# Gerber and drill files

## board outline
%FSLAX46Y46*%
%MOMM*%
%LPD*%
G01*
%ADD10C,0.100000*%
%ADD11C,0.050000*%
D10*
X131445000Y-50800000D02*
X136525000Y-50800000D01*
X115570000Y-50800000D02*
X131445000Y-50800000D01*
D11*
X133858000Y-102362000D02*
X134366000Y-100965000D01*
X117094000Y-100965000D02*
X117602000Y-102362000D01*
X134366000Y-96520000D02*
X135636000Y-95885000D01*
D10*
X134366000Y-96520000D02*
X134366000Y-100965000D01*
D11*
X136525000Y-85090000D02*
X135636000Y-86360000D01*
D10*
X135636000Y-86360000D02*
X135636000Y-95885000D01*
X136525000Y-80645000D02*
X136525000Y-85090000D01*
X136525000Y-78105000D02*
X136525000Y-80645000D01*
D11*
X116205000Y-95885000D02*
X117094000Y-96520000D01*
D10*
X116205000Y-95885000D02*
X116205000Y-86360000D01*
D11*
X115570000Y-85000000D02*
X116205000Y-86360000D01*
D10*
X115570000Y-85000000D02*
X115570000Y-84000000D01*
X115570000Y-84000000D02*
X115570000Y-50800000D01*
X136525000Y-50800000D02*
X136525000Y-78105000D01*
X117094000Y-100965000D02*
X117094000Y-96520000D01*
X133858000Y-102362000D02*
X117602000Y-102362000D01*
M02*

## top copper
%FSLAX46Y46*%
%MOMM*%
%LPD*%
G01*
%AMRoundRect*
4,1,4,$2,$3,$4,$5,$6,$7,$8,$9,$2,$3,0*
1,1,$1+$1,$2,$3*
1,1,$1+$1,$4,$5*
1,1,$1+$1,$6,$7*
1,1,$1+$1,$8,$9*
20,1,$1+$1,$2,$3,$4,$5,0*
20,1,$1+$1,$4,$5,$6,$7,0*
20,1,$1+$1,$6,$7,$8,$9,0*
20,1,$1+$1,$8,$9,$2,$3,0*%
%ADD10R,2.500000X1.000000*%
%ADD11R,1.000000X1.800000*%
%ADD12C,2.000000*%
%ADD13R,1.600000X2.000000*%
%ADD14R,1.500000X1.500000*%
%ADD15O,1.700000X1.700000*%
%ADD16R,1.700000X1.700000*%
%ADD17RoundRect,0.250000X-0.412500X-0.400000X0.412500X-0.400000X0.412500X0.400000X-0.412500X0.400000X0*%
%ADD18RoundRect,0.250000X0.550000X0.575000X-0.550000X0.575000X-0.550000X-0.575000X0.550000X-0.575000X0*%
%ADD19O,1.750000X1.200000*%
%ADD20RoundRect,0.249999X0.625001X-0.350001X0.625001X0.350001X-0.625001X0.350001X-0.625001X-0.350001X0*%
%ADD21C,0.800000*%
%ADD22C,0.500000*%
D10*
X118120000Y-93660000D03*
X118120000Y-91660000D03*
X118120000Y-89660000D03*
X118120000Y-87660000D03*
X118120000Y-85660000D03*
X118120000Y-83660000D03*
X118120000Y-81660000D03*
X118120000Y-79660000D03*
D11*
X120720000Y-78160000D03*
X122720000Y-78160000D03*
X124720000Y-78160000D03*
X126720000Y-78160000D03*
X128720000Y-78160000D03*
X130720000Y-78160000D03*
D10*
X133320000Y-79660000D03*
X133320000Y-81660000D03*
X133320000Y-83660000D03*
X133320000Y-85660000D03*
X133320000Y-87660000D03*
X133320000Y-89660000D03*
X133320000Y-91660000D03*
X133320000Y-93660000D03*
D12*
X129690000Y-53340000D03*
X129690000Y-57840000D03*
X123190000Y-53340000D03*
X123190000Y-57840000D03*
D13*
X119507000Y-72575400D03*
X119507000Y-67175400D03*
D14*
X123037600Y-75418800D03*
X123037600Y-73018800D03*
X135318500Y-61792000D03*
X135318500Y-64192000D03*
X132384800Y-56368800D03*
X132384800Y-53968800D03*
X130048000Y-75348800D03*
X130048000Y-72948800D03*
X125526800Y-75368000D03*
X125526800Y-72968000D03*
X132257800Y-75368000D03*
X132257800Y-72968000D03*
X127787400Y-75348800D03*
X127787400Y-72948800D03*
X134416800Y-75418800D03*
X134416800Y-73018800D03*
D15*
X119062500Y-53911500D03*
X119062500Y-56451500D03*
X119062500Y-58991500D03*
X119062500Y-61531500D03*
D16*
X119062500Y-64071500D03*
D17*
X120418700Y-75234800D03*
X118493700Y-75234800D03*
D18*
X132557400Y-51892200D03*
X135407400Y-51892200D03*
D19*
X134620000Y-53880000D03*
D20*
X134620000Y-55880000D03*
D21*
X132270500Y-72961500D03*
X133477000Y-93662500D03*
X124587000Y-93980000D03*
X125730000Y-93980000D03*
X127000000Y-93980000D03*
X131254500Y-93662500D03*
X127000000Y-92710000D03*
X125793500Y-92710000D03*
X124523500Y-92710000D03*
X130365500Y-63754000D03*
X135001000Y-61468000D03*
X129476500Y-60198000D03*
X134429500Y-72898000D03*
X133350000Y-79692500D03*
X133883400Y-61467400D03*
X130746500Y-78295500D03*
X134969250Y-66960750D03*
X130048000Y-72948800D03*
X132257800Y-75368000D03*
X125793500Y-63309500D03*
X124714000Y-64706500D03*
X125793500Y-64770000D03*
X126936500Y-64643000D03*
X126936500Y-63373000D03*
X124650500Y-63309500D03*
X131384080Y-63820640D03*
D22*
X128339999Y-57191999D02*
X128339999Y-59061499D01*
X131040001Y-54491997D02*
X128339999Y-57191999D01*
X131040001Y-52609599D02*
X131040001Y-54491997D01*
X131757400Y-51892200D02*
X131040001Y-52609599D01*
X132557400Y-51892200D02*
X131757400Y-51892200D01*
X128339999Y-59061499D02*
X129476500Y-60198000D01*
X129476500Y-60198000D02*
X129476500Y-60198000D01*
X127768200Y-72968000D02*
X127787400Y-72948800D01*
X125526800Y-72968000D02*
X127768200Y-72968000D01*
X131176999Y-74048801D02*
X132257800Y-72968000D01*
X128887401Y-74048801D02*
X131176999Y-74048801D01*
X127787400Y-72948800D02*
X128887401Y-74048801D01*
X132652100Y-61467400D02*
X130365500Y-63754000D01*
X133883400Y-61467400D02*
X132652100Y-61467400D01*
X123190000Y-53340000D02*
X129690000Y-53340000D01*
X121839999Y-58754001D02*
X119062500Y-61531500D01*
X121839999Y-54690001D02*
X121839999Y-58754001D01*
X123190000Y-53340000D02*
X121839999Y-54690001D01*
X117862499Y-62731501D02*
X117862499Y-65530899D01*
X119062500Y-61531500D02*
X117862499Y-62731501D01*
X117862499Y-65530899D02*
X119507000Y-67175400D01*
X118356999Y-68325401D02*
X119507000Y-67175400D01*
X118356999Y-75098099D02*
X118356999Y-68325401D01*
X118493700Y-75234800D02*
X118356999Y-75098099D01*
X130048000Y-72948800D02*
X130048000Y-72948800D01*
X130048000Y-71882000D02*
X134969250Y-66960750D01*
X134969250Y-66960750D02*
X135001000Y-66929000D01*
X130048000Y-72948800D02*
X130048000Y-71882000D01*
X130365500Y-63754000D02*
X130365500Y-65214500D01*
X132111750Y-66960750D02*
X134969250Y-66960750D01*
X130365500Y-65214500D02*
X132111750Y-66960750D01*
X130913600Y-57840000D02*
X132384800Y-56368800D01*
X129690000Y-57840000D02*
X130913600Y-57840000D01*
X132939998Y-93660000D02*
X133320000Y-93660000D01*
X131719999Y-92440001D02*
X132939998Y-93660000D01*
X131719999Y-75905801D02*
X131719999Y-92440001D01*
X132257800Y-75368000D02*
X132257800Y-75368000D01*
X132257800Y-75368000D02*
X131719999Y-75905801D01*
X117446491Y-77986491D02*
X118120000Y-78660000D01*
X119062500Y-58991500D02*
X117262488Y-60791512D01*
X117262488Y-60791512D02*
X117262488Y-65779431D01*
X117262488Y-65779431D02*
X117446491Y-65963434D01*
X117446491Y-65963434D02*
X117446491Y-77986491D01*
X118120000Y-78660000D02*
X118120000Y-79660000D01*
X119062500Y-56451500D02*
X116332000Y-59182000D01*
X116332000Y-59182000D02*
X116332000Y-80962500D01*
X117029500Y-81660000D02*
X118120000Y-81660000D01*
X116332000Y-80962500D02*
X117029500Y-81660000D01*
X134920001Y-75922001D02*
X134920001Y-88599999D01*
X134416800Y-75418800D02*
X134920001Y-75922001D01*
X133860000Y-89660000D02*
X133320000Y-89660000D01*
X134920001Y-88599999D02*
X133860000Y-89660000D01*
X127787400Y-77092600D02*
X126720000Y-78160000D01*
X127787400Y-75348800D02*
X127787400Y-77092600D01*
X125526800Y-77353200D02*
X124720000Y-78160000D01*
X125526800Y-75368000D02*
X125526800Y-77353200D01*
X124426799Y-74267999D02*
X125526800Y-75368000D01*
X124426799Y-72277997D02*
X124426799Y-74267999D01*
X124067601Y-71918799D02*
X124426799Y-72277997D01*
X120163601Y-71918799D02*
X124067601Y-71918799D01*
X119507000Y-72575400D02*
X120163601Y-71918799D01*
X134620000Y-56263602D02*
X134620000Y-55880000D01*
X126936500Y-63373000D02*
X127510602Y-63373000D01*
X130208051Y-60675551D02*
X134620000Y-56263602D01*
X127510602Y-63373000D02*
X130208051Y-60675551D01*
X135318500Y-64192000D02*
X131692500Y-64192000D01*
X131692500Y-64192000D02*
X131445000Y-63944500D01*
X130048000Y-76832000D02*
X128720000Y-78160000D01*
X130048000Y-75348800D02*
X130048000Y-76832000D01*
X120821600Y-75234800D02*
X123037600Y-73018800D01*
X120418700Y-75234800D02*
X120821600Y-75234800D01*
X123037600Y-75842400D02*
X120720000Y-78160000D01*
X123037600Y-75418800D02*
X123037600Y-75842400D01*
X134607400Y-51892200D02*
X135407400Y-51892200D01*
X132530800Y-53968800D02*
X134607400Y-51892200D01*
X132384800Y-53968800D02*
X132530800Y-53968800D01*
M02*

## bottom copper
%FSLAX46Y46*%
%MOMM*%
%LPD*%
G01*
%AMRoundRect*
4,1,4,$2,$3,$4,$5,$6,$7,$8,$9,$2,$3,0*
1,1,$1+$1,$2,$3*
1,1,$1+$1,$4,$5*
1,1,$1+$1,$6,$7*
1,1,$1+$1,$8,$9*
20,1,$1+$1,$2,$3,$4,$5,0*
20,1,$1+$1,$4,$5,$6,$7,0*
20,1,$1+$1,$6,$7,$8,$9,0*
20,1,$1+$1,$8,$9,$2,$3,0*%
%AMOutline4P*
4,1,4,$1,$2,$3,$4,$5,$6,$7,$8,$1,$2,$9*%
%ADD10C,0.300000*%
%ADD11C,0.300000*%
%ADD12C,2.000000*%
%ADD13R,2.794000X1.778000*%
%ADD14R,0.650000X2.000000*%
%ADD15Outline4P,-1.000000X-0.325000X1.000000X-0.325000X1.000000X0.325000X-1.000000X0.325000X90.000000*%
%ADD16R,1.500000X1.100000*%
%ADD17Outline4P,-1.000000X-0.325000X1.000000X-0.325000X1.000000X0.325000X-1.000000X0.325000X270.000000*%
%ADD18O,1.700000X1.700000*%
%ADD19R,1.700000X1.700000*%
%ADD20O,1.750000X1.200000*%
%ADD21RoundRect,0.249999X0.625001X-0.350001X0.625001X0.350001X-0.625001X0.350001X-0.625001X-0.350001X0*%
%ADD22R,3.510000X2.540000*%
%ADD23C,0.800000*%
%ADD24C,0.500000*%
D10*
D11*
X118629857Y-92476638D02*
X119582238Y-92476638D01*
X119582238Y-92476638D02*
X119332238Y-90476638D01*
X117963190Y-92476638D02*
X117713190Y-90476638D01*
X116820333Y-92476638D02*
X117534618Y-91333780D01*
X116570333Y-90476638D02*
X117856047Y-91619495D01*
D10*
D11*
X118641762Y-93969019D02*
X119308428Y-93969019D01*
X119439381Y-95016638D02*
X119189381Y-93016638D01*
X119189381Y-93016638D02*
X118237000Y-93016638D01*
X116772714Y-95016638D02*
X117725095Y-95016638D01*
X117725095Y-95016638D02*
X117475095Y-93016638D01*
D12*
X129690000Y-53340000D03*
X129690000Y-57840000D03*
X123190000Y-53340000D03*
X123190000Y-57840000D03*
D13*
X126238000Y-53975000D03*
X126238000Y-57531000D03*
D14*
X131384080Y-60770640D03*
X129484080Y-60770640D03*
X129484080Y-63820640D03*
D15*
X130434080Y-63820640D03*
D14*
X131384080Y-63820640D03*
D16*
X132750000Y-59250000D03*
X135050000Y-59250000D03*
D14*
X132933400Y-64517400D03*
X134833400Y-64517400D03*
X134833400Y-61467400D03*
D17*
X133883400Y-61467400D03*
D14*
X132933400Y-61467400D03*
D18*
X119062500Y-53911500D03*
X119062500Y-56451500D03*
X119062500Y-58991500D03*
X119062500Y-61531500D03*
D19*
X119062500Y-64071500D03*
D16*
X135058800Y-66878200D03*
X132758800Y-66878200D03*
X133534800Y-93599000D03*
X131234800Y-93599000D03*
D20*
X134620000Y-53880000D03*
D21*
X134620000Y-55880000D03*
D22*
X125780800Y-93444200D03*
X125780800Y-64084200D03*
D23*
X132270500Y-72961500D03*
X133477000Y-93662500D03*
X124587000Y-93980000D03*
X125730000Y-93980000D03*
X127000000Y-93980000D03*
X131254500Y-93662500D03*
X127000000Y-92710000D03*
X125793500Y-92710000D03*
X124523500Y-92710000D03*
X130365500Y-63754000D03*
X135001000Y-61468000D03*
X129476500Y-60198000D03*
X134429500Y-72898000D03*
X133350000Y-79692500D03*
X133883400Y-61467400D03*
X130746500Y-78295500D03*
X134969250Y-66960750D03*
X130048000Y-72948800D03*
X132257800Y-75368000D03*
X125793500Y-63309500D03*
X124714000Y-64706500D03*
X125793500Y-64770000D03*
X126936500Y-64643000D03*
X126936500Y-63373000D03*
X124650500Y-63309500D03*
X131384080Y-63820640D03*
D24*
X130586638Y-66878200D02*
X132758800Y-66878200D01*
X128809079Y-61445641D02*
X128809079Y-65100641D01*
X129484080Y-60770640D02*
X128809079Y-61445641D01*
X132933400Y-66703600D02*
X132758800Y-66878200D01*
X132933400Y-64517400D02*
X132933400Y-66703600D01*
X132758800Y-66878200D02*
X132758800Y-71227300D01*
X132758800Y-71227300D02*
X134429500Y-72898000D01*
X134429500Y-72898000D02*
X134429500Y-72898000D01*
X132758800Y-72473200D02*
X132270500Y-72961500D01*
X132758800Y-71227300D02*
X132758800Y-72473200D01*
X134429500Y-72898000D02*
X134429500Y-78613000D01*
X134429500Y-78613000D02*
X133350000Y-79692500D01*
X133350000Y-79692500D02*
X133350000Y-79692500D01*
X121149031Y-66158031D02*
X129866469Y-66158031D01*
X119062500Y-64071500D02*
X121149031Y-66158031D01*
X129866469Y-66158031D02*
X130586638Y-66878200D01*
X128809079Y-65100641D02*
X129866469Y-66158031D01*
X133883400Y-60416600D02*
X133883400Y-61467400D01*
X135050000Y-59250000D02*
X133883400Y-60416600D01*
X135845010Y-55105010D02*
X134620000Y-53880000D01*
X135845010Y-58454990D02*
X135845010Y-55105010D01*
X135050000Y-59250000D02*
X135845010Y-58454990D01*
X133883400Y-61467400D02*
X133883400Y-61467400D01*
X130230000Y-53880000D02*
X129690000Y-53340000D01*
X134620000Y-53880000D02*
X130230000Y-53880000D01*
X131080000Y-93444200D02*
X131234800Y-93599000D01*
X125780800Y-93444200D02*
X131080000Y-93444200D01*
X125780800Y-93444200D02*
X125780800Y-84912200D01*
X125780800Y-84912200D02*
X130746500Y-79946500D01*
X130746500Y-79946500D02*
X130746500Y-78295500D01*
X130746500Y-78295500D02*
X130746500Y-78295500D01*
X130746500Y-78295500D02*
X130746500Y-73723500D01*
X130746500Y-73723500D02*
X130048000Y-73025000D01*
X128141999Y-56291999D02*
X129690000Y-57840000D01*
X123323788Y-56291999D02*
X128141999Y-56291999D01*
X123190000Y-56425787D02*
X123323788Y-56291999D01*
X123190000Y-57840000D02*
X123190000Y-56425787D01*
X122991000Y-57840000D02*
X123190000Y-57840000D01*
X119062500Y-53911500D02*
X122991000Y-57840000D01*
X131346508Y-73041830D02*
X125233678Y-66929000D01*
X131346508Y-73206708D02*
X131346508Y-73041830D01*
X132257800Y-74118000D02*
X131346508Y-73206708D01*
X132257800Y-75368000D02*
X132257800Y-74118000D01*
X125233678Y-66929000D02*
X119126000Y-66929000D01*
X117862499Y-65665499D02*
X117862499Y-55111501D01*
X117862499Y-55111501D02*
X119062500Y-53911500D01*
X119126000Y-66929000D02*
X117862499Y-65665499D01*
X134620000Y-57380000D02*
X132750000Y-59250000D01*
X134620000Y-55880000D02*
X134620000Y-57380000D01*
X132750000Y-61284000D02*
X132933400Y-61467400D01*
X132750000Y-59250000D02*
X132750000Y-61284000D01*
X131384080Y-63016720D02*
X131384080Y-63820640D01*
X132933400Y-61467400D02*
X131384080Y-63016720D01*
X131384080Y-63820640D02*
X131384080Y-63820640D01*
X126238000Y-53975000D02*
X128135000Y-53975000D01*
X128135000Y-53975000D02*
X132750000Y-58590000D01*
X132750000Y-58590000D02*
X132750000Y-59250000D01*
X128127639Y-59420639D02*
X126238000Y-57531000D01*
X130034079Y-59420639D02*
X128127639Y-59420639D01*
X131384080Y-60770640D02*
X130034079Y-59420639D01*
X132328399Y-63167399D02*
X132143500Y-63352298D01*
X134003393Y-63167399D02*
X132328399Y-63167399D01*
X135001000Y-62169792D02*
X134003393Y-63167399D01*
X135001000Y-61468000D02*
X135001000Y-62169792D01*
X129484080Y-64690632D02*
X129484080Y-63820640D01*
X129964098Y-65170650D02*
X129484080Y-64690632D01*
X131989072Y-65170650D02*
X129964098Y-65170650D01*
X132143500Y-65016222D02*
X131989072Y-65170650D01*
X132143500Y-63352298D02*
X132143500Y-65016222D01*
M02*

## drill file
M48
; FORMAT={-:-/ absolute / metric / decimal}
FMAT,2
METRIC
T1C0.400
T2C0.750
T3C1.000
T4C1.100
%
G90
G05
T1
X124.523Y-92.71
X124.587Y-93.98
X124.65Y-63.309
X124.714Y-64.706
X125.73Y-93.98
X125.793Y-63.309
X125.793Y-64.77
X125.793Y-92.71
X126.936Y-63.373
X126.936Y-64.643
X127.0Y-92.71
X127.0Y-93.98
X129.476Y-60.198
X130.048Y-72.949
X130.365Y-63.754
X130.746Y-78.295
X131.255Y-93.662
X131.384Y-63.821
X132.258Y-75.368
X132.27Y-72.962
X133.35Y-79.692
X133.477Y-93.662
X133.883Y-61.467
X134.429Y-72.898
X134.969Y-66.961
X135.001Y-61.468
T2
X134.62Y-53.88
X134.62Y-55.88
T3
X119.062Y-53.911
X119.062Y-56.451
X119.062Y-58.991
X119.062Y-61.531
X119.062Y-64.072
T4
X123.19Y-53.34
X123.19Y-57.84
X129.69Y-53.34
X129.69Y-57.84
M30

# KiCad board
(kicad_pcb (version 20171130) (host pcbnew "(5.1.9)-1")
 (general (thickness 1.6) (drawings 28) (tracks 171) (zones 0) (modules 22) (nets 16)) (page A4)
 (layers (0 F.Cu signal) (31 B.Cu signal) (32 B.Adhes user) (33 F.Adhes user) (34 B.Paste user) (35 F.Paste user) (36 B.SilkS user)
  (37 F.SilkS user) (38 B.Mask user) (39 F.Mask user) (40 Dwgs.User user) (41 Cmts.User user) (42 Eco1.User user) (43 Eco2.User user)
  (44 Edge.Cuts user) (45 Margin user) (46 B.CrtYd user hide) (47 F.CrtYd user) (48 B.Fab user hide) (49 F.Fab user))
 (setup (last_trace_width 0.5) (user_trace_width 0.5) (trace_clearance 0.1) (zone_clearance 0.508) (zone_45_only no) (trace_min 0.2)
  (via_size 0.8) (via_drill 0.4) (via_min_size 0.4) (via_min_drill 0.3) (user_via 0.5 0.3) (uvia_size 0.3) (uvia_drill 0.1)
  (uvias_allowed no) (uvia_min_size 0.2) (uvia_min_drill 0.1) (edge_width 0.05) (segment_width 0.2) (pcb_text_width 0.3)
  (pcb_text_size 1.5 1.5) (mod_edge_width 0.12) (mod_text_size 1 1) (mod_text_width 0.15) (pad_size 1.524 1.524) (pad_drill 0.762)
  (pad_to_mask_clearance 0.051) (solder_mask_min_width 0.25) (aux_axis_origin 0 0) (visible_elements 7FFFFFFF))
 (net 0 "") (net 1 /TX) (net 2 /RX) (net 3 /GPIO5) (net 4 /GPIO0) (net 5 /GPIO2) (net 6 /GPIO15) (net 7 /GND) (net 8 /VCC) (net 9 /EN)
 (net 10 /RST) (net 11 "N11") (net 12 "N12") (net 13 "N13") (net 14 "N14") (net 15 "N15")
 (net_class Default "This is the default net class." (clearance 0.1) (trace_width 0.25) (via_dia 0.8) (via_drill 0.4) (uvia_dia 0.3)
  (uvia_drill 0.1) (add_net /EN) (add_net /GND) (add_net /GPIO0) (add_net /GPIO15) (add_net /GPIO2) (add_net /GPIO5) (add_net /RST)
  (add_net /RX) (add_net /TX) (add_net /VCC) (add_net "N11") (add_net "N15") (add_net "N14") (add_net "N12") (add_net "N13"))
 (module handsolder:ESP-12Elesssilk (layer F.Cu) (at 125.72 90.16 180)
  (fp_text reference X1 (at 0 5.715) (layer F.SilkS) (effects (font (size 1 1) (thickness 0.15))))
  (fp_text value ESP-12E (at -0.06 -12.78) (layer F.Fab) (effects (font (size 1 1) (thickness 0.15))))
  (pad 22 smd rect (at 7.6 -3.5 180) (size 2.5 1) (layers F.Cu F.Paste F.Mask))
  (pad 21 smd rect (at 7.6 -1.5 180) (size 2.5 1) (layers F.Cu F.Paste F.Mask))
  (pad 20 smd rect (at 7.6 0.5 180) (size 2.5 1) (layers F.Cu F.Paste F.Mask))
  (pad 19 smd rect (at 7.6 2.5 180) (size 2.5 1) (layers F.Cu F.Paste F.Mask))
  (pad 18 smd rect (at 7.6 4.5 180) (size 2.5 1) (layers F.Cu F.Paste F.Mask))
  (pad 17 smd rect (at 7.6 6.5 180) (size 2.5 1) (layers F.Cu F.Paste F.Mask))
  (pad 16 smd rect (at 7.6 8.5 180) (size 2.5 1) (layers F.Cu F.Paste F.Mask) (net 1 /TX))
  (pad 15 smd rect (at 7.6 10.5 180) (size 2.5 1) (layers F.Cu F.Paste F.Mask) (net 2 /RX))
  (pad 14 smd rect (at 5 12 180) (size 1 1.8) (layers F.Cu F.Paste F.Mask) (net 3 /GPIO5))
  (pad 13 smd rect (at 3 12 180) (size 1 1.8) (layers F.Cu F.Paste F.Mask))
  (pad 12 smd rect (at 1 12 180) (size 1 1.8) (layers F.Cu F.Paste F.Mask) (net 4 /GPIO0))
  (pad 11 smd rect (at -1 12 180) (size 1 1.8) (layers F.Cu F.Paste F.Mask) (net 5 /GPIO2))
  (pad 10 smd rect (at -3 12 180) (size 1 1.8) (layers F.Cu F.Paste F.Mask) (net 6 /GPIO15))
  (pad 9 smd rect (at -5 12 180) (size 1 1.8) (layers F.Cu F.Paste F.Mask) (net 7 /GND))
  (pad 8 smd rect (at -7.6 10.5 180) (size 2.5 1) (layers F.Cu F.Paste F.Mask) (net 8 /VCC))
  (pad 7 smd rect (at -7.6 8.5 180) (size 2.5 1) (layers F.Cu F.Paste F.Mask))
  (pad 6 smd rect (at -7.6 6.5 180) (size 2.5 1) (layers F.Cu F.Paste F.Mask))
  (pad 5 smd rect (at -7.6 4.5 180) (size 2.5 1) (layers F.Cu F.Paste F.Mask))
  (pad 4 smd rect (at -7.6 2.5 180) (size 2.5 1) (layers F.Cu F.Paste F.Mask))
  (pad 3 smd rect (at -7.6 0.5 180) (size 2.5 1) (layers F.Cu F.Paste F.Mask) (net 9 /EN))
  (pad 2 smd rect (at -7.6 -1.5 180) (size 2.5 1) (layers F.Cu F.Paste F.Mask))
  (pad 1 smd rect (at -7.6 -3.5 180) (size 2.5 1) (layers F.Cu F.Paste F.Mask) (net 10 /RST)))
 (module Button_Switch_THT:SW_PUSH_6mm (layer F.Cu) (at 123.19 53.34)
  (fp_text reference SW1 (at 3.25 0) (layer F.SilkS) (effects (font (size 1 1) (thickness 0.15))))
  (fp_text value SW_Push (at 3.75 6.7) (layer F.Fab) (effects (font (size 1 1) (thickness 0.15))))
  (pad 1 thru_hole circle (at 6.5 0 90) (size 2 2) (drill 1.1) (layers *.Cu *.Mask) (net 7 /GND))
  (pad 2 thru_hole circle (at 6.5 4.5 90) (size 2 2) (drill 1.1) (layers *.Cu *.Mask) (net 10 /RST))
  (pad 1 thru_hole circle (at 0 0 90) (size 2 2) (drill 1.1) (layers *.Cu *.Mask) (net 7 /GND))
  (pad 2 thru_hole circle (at 0 4.5 90) (size 2 2) (drill 1.1) (layers *.Cu *.Mask) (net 10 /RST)))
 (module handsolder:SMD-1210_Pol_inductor (layer B.Cu) (at 126.238 55.753 270)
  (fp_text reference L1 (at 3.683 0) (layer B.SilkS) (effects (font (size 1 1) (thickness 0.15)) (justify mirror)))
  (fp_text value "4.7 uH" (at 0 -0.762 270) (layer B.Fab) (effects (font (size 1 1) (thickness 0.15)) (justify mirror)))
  (pad 1 smd rect (at -1.778 0 270) (size 1.778 2.794) (layers B.Cu B.Paste B.Mask) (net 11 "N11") (zone_connect 2))
  (pad 2 smd rect (at 1.778 0 270) (size 1.778 2.794) (layers B.Cu B.Paste B.Mask) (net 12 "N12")))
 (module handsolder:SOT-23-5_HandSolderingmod (layer B.Cu) (at 130.43408 62.27064 90)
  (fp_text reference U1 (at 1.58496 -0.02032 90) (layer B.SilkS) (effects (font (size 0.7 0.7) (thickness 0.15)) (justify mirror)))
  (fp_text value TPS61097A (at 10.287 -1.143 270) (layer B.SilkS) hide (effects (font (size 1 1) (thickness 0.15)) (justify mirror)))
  (pad 5 smd rect (at 1.5 0.95 90) (size 2 0.65) (layers B.Cu B.Paste B.Mask) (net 12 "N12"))
  (pad 4 smd rect (at 1.5 -0.95 90) (size 2 0.65) (layers B.Cu B.Paste B.Mask) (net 8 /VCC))
  (pad 3 smd rect (at -1.55 -0.95 90) (size 2 0.65) (layers B.Cu B.Paste B.Mask) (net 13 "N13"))
  (pad 2 smd trapezoid (at -1.55 0 90) (size 2 0.65) (layers B.Cu B.Paste B.Mask) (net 7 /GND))
  (pad 1 smd rect (at -1.55 0.95 90) (size 2 0.65) (layers B.Cu B.Paste B.Mask) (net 11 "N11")))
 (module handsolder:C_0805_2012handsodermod (layer B.Cu) (at 133.9 59.25 180)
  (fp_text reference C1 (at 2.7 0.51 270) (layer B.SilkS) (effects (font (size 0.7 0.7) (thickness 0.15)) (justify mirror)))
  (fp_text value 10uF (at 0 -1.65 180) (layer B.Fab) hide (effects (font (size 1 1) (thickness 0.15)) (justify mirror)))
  (pad 2 smd rect (at 1.15 0 180) (size 1.5 1.1) (layers B.Cu B.Paste B.Mask) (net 11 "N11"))
  (pad 1 smd rect (at -1.15 0 180) (size 1.5 1.1) (layers B.Cu B.Paste B.Mask) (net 7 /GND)))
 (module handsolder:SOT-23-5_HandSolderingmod (layer B.Cu) (at 133.8834 63.0174 270)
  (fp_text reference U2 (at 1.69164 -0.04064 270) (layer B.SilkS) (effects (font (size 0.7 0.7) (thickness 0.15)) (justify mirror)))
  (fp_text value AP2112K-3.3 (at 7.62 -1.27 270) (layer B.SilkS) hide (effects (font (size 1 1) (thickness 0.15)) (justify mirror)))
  (pad 5 smd rect (at 1.5 0.95 270) (size 2 0.65) (layers B.Cu B.Paste B.Mask) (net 8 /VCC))
  (pad 4 smd rect (at 1.5 -0.95 270) (size 2 0.65) (layers B.Cu B.Paste B.Mask))
  (pad 3 smd rect (at -1.55 -0.95 270) (size 2 0.65) (layers B.Cu B.Paste B.Mask) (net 13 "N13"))
  (pad 2 smd trapezoid (at -1.55 0 270) (size 2 0.65) (layers B.Cu B.Paste B.Mask) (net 7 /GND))
  (pad 1 smd rect (at -1.55 0.95 270) (size 2 0.65) (layers B.Cu B.Paste B.Mask) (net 11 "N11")))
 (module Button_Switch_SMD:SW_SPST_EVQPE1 (layer F.Cu) (at 119.507 69.8754 90)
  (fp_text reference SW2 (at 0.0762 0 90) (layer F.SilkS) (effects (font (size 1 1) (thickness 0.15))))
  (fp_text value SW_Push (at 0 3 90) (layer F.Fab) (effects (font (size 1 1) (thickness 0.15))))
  (pad 1 smd rect (at -2.7 0 90) (size 2 1.6) (layers F.Cu F.Paste F.Mask) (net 4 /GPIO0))
  (pad 2 smd rect (at 2.7 0 90) (size 2 1.6) (layers F.Cu F.Paste F.Mask) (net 7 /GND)))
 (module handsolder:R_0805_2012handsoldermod (layer F.Cu) (at 123.0376 74.2188 270)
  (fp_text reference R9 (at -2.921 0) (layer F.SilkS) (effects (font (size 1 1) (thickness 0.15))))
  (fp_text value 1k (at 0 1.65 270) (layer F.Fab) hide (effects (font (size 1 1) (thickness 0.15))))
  (pad 2 smd rect (at 1.2 0 270) (size 1.5 1.5) (layers F.Cu F.Paste F.Mask) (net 3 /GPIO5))
  (pad 1 smd rect (at -1.2 0 270) (size 1.5 1.5) (layers F.Cu F.Paste F.Mask) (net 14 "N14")))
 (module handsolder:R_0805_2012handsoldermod (layer F.Cu) (at 135.3185 62.992 90)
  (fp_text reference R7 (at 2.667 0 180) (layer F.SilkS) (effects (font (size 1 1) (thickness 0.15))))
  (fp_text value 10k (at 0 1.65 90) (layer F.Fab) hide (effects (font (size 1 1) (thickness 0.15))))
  (pad 2 smd rect (at 1.2 0 90) (size 1.5 1.5) (layers F.Cu F.Paste F.Mask) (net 13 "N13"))
  (pad 1 smd rect (at -1.2 0 90) (size 1.5 1.5) (layers F.Cu F.Paste F.Mask) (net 11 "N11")))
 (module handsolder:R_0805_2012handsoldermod (layer F.Cu) (at 132.3848 55.1688 270)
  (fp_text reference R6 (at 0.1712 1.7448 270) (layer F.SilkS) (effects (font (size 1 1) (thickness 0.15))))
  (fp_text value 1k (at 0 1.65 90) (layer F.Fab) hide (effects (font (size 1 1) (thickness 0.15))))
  (pad 2 smd rect (at 1.2 0 270) (size 1.5 1.5) (layers F.Cu F.Paste F.Mask) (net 10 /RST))
  (pad 1 smd rect (at -1.2 0 270) (size 1.5 1.5) (layers F.Cu F.Paste F.Mask) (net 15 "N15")))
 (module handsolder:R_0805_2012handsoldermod (layer F.Cu) (at 130.048 74.1488 270)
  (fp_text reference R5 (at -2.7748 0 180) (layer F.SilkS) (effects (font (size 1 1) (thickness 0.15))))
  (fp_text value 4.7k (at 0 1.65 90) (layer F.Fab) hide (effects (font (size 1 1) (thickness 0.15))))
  (pad 2 smd rect (at 1.2 0 270) (size 1.5 1.5) (layers F.Cu F.Paste F.Mask) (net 6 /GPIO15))
  (pad 1 smd rect (at -1.2 0 270) (size 1.5 1.5) (layers F.Cu F.Paste F.Mask) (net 7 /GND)))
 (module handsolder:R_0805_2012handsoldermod (layer F.Cu) (at 125.5268 74.168 270)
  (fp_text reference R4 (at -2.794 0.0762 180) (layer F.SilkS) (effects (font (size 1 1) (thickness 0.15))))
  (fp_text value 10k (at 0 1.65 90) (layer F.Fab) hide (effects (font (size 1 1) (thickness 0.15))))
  (pad 2 smd rect (at 1.2 0 270) (size 1.5 1.5) (layers F.Cu F.Paste F.Mask) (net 4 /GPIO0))
  (pad 1 smd rect (at -1.2 0 270) (size 1.5 1.5) (layers F.Cu F.Paste F.Mask) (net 8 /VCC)))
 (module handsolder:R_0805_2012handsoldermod (layer F.Cu) (at 132.2578 74.168 270)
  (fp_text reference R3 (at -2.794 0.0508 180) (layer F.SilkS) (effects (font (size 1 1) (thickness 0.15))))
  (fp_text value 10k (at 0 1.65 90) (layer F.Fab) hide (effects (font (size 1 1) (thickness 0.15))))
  (pad 2 smd rect (at 1.2 0 270) (size 1.5 1.5) (layers F.Cu F.Paste F.Mask) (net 10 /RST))
  (pad 1 smd rect (at -1.2 0 270) (size 1.5 1.5) (layers F.Cu F.Paste F.Mask) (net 8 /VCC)))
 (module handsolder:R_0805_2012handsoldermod (layer F.Cu) (at 127.7874 74.1488 270)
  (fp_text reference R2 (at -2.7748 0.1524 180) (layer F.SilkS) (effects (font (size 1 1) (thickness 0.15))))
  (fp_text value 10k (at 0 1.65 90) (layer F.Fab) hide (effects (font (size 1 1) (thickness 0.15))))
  (pad 2 smd rect (at 1.2 0 270) (size 1.5 1.5) (layers F.Cu F.Paste F.Mask) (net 5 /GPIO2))
  (pad 1 smd rect (at -1.2 0 270) (size 1.5 1.5) (layers F.Cu F.Paste F.Mask) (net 8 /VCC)))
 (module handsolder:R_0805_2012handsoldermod (layer F.Cu) (at 134.4168 74.2188 270)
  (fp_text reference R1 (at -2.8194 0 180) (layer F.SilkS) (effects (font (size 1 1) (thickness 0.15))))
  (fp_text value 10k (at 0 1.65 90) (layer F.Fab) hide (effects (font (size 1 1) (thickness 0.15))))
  (pad 2 smd rect (at 1.2 0 270) (size 1.5 1.5) (layers F.Cu F.Paste F.Mask) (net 9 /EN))
  (pad 1 smd rect (at -1.2 0 270) (size 1.5 1.5) (layers F.Cu F.Paste F.Mask) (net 8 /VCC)))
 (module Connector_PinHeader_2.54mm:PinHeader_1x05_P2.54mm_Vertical (layer F.Cu) (at 119.0625 64.0715 180)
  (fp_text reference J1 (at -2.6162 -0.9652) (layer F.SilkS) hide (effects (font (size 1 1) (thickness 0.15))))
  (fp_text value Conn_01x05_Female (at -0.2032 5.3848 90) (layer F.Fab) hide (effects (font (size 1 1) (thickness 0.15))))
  (pad 5 thru_hole oval (at 0 10.16 180) (size 1.7 1.7) (drill 1) (layers *.Cu *.Mask) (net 10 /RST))
  (pad 4 thru_hole oval (at 0 7.62 180) (size 1.7 1.7) (drill 1) (layers *.Cu *.Mask) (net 1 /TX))
  (pad 3 thru_hole oval (at 0 5.08 180) (size 1.7 1.7) (drill 1) (layers *.Cu *.Mask) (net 2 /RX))
  (pad 2 thru_hole oval (at 0 2.54 180) (size 1.7 1.7) (drill 1) (layers *.Cu *.Mask) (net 7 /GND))
  (pad 1 thru_hole rect (at 0 0 180) (size 1.7 1.7) (drill 1) (layers *.Cu *.Mask) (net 8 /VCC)))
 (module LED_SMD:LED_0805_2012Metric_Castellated (layer F.Cu) (at 119.4562 75.2348)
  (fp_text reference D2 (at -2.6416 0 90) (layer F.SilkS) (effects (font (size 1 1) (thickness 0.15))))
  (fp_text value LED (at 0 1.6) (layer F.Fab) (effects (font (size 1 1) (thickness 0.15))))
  (pad 2 smd roundrect (at 0.9625 0) (size 1.325 1.3) (layers F.Cu F.Paste F.Mask) (roundrect_rratio 0.1923076923076923) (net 14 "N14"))
  (pad 1 smd roundrect (at -0.9625 0) (size 1.325 1.3) (layers F.Cu F.Paste F.Mask) (roundrect_rratio 0.1923076923076923) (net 7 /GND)))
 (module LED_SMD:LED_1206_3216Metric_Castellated (layer F.Cu) (at 133.9824 51.8922 180)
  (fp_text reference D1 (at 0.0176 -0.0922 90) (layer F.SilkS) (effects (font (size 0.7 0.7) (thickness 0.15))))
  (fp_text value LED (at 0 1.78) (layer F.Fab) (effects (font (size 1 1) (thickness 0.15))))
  (pad 2 smd roundrect (at 1.425 0 180) (size 1.6 1.65) (layers F.Cu F.Paste F.Mask) (roundrect_rratio 0.15625) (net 8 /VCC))
  (pad 1 smd roundrect (at -1.425 0 180) (size 1.6 1.65) (layers F.Cu F.Paste F.Mask) (roundrect_rratio 0.15625) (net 15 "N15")))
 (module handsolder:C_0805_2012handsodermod (layer B.Cu) (at 133.9088 66.8782)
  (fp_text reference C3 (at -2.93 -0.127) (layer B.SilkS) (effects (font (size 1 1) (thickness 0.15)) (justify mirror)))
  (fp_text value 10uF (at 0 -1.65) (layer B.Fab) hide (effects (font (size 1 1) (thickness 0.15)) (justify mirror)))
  (pad 2 smd rect (at 1.15 0) (size 1.5 1.1) (layers B.Cu B.Paste B.Mask) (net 7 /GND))
  (pad 1 smd rect (at -1.15 0) (size 1.5 1.1) (layers B.Cu B.Paste B.Mask) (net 8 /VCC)))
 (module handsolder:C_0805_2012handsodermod (layer B.Cu) (at 132.3848 93.599)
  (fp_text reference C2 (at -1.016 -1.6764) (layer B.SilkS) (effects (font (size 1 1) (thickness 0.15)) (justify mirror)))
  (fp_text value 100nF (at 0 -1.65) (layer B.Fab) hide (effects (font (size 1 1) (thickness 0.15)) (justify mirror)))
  (pad 2 smd rect (at 1.15 0) (size 1.5 1.1) (layers B.Cu B.Paste B.Mask) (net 10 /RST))
  (pad 1 smd rect (at -1.15 0) (size 1.5 1.1) (layers B.Cu B.Paste B.Mask) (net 7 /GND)))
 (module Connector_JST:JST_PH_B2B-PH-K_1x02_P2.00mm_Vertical (layer B.Cu) (at 134.62 55.88 90)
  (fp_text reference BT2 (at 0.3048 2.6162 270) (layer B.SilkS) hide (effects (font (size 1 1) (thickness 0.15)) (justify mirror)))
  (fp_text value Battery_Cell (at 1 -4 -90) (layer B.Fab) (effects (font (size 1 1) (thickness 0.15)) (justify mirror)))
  (pad 2 thru_hole oval (at 2 0 90) (size 1.2 1.75) (drill 0.75) (layers *.Cu *.Mask) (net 7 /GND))
  (pad 1 thru_hole roundrect (at 0 0 90) (size 1.2 1.75) (drill 0.75) (layers *.Cu *.Mask) (roundrect_rratio 0.2083325) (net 11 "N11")))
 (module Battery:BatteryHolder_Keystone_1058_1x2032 (layer B.Cu) (at 125.7808 78.7642 270)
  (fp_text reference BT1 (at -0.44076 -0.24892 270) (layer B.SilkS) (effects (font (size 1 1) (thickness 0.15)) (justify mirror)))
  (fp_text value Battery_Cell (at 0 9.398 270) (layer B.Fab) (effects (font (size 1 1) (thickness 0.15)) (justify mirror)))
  (pad 2 smd rect (at 14.68 0 270) (size 2.54 3.51) (layers B.Cu B.Paste B.Mask) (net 7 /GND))
  (pad 1 smd rect (at -14.68 0 270) (size 2.54 3.51) (layers B.Cu B.Paste B.Mask) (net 11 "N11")))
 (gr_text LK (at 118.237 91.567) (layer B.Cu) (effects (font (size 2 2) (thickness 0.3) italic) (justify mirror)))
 (gr_line (start 131.445 50.8) (end 136.525 50.8) (layer Edge.Cuts) (width 0.1))
 (gr_line (start 115.57 50.8) (end 131.445 50.8) (layer Edge.Cuts) (width 0.1))
 (gr_line (start 133.858 102.362) (end 134.366 100.965) (layer Edge.Cuts) (width 0.05))
 (gr_line (start 117.094 100.965) (end 117.602 102.362) (layer Edge.Cuts) (width 0.05))
 (gr_line (start 134.366 96.52) (end 135.636 95.885) (layer Edge.Cuts) (width 0.05))
 (gr_line (start 134.366 96.52) (end 134.366 100.965) (layer Edge.Cuts) (width 0.1))
 (gr_line (start 136.525 85.09) (end 135.636 86.36) (layer Edge.Cuts) (width 0.05))
 (gr_line (start 135.636 86.36) (end 135.636 95.885) (layer Edge.Cuts) (width 0.1))
 (gr_line (start 136.525 80.645) (end 136.525 85.09) (layer Edge.Cuts) (width 0.1))
 (gr_line (start 136.525 78.105) (end 136.525 80.645) (layer Edge.Cuts) (width 0.1))
 (gr_line (start 116.205 95.885) (end 117.094 96.52) (layer Edge.Cuts) (width 0.05))
 (gr_line (start 116.205 95.885) (end 116.205 86.36) (layer Edge.Cuts) (width 0.1))
 (gr_line (start 115.57 85) (end 116.205 86.36) (layer Edge.Cuts) (width 0.05))
 (gr_line (start 115.57 85) (end 115.57 84) (layer Edge.Cuts) (width 0.1))
 (gr_line (start 115.57 84) (end 115.57 50.8) (layer Edge.Cuts) (width 0.1))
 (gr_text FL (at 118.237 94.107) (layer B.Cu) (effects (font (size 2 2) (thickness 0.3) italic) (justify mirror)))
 (gr_line (start 136.525 50.8) (end 136.525 78.105) (layer Edge.Cuts) (width 0.1))
 (gr_line (start 117.094 100.965) (end 117.094 96.52) (layer Edge.Cuts) (width 0.1))
 (gr_line (start 133.858 102.362) (end 117.602 102.362) (layer Edge.Cuts) (width 0.1))
 (via (at 132.2705 72.9615) (size 0.8) (drill 0.4) (layers F.Cu B.Cu) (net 8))
 (via (at 133.477 93.6625) (size 0.8) (drill 0.4) (layers F.Cu B.Cu) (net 10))
 (via (at 124.587 93.98) (size 0.8) (drill 0.4) (layers F.Cu B.Cu) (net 7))
 (via (at 125.73 93.98) (size 0.8) (drill 0.4) (layers F.Cu B.Cu) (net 7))
 (via (at 127 93.98) (size 0.8) (drill 0.4) (layers F.Cu B.Cu) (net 7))
 (via (at 131.2545 93.6625) (size 0.8) (drill 0.4) (layers F.Cu B.Cu) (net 7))
 (via (at 127 92.71) (size 0.8) (drill 0.4) (layers F.Cu B.Cu) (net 7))
 (via (at 125.7935 92.71) (size 0.8) (drill 0.4) (layers F.Cu B.Cu) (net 7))
 (via (at 124.5235 92.71) (size 0.8) (drill 0.4) (layers F.Cu B.Cu) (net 7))
 (via (at 130.3655 63.754) (size 0.8) (drill 0.4) (layers F.Cu B.Cu) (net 7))
 (via (at 135.001 61.468) (size 0.8) (drill 0.4) (layers F.Cu B.Cu) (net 13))
 (segment (start 130.586638 66.8782) (end 132.7588 66.8782) (width 0.5) (layer B.Cu) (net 8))
 (segment (start 128.809079 61.445641) (end 128.809079 65.100641) (width 0.5) (layer B.Cu) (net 8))
 (segment (start 129.48408 60.77064) (end 128.809079 61.445641) (width 0.5) (layer B.Cu) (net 8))
 (segment (start 132.9334 66.7036) (end 132.7588 66.8782) (width 0.5) (layer B.Cu) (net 8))
 (segment (start 132.9334 64.5174) (end 132.9334 66.7036) (width 0.5) (layer B.Cu) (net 8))
 (segment (start 128.339999 57.191999) (end 128.339999 59.061499) (width 0.5) (layer F.Cu) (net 8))
 (segment (start 131.040001 54.491997) (end 128.339999 57.191999) (width 0.5) (layer F.Cu) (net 8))
 (segment (start 131.040001 52.609599) (end 131.040001 54.491997) (width 0.5) (layer F.Cu) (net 8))
 (segment (start 131.7574 51.8922) (end 131.040001 52.609599) (width 0.5) (layer F.Cu) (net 8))
 (segment (start 132.5574 51.8922) (end 131.7574 51.8922) (width 0.5) (layer F.Cu) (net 8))
 (segment (start 128.339999 59.061499) (end 129.4765 60.198) (width 0.5) (layer F.Cu) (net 8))
 (segment (start 129.4765 60.198) (end 129.4765 60.198) (width 0.5) (layer F.Cu) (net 8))
 (via (at 129.4765 60.198) (size 0.8) (drill 0.4) (layers F.Cu B.Cu) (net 8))
 (segment (start 132.7588 66.8782) (end 132.7588 71.2273) (width 0.5) (layer B.Cu) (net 8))
 (segment (start 132.7588 71.2273) (end 134.4295 72.898) (width 0.5) (layer B.Cu) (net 8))
 (segment (start 134.4295 72.898) (end 134.4295 72.898) (width 0.5) (layer B.Cu) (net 8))
 (via (at 134.4295 72.898) (size 0.8) (drill 0.4) (layers F.Cu B.Cu) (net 8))
 (segment (start 132.7588 72.4732) (end 132.2705 72.9615) (width 0.5) (layer B.Cu) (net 8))
 (segment (start 132.7588 71.2273) (end 132.7588 72.4732) (width 0.5) (layer B.Cu) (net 8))
 (segment (start 134.4295 72.898) (end 134.4295 78.613) (width 0.5) (layer B.Cu) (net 8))
 (segment (start 134.4295 78.613) (end 133.35 79.6925) (width 0.5) (layer B.Cu) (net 8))
 (segment (start 133.35 79.6925) (end 133.35 79.6925) (width 0.5) (layer B.Cu) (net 8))
 (via (at 133.35 79.6925) (size 0.8) (drill 0.4) (layers F.Cu B.Cu) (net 8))
 (segment (start 127.7682 72.968) (end 127.7874 72.9488) (width 0.5) (layer F.Cu) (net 8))
 (segment (start 125.5268 72.968) (end 127.7682 72.968) (width 0.5) (layer F.Cu) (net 8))
 (segment (start 131.176999 74.048801) (end 132.2578 72.968) (width 0.5) (layer F.Cu) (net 8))
 (segment (start 128.887401 74.048801) (end 131.176999 74.048801) (width 0.5) (layer F.Cu) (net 8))
 (segment (start 127.7874 72.9488) (end 128.887401 74.048801) (width 0.5) (layer F.Cu) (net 8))
 (segment (start 121.149031 66.158031) (end 129.866469 66.158031) (width 0.5) (layer B.Cu) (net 8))
 (segment (start 119.0625 64.0715) (end 121.149031 66.158031) (width 0.5) (layer B.Cu) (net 8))
 (segment (start 129.866469 66.158031) (end 130.586638 66.8782) (width 0.5) (layer B.Cu) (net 8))
 (segment (start 128.809079 65.100641) (end 129.866469 66.158031) (width 0.5) (layer B.Cu) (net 8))
 (segment (start 133.8834 60.4166) (end 133.8834 61.4674) (width 0.5) (layer B.Cu) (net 7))
 (segment (start 135.05 59.25) (end 133.8834 60.4166) (width 0.5) (layer B.Cu) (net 7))
 (segment (start 135.84501 55.10501) (end 134.62 53.88) (width 0.5) (layer B.Cu) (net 7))
 (segment (start 135.84501 58.45499) (end 135.84501 55.10501) (width 0.5) (layer B.Cu) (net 7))
 (segment (start 135.05 59.25) (end 135.84501 58.45499) (width 0.5) (layer B.Cu) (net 7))
 (segment (start 133.8834 61.4674) (end 133.8834 61.4674) (width 0.5) (layer B.Cu) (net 7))
 (via (at 133.8834 61.4674) (size 0.8) (drill 0.4) (layers F.Cu B.Cu) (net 7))
 (segment (start 132.6521 61.4674) (end 130.3655 63.754) (width 0.5) (layer F.Cu) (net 7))
 (segment (start 133.8834 61.4674) (end 132.6521 61.4674) (width 0.5) (layer F.Cu) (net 7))
 (segment (start 123.19 53.34) (end 129.69 53.34) (width 0.5) (layer F.Cu) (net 7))
 (segment (start 130.23 53.88) (end 129.69 53.34) (width 0.5) (layer B.Cu) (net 7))
 (segment (start 134.62 53.88) (end 130.23 53.88) (width 0.5) (layer B.Cu) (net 7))
 (segment (start 121.839999 58.754001) (end 119.0625 61.5315) (width 0.5) (layer F.Cu) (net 7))
 (segment (start 121.839999 54.690001) (end 121.839999 58.754001) (width 0.5) (layer F.Cu) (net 7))
 (segment (start 123.19 53.34) (end 121.839999 54.690001) (width 0.5) (layer F.Cu) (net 7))
 (segment (start 117.862499 62.731501) (end 117.862499 65.530899) (width 0.5) (layer F.Cu) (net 7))
 (segment (start 119.0625 61.5315) (end 117.862499 62.731501) (width 0.5) (layer F.Cu) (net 7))
 (segment (start 117.862499 65.530899) (end 119.507 67.1754) (width 0.5) (layer F.Cu) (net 7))
 (segment (start 131.08 93.4442) (end 131.2348 93.599) (width 0.5) (layer B.Cu) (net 7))
 (segment (start 125.7808 93.4442) (end 131.08 93.4442) (width 0.5) (layer B.Cu) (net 7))
 (segment (start 125.7808 93.4442) (end 125.7808 84.9122) (width 0.5) (layer B.Cu) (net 7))
 (segment (start 125.7808 84.9122) (end 130.7465 79.9465) (width 0.5) (layer B.Cu) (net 7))
 (segment (start 130.7465 79.9465) (end 130.7465 78.2955) (width 0.5) (layer B.Cu) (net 7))
 (segment (start 130.7465 78.2955) (end 130.7465 78.2955) (width 0.5) (layer B.Cu) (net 7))
 (via (at 130.7465 78.2955) (size 0.8) (drill 0.4) (layers F.Cu B.Cu) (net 7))
 (segment (start 118.356999 68.325401) (end 119.507 67.1754) (width 0.5) (layer F.Cu) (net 7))
 (segment (start 118.356999 75.098099) (end 118.356999 68.325401) (width 0.5) (layer F.Cu) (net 7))
 (segment (start 118.4937 75.2348) (end 118.356999 75.098099) (width 0.5) (layer F.Cu) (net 7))
 (segment (start 130.048 72.9488) (end 130.048 72.9488) (width 0.5) (layer F.Cu) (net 7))
 (segment (start 130.048 71.882) (end 134.96925 66.96075) (width 0.5) (layer F.Cu) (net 7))
 (segment (start 134.96925 66.96075) (end 135.001 66.929) (width 0.5) (layer F.Cu) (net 7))
 (via (at 134.96925 66.96075) (size 0.8) (drill 0.4) (layers F.Cu B.Cu) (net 7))
 (segment (start 130.7465 78.2955) (end 130.7465 73.7235) (width 0.5) (layer B.Cu) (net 7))
 (segment (start 130.7465 73.7235) (end 130.048 73.025) (width 0.5) (layer B.Cu) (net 7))
 (segment (start 130.048 72.9488) (end 130.048 71.882) (width 0.5) (layer F.Cu) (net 7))
 (via (at 130.048 72.9488) (size 0.8) (drill 0.4) (layers F.Cu B.Cu) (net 7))
 (segment (start 130.3655 63.754) (end 130.3655 65.2145) (width 0.5) (layer F.Cu) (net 7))
 (segment (start 132.11175 66.96075) (end 134.96925 66.96075) (width 0.5) (layer F.Cu) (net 7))
 (segment (start 130.3655 65.2145) (end 132.11175 66.96075) (width 0.5) (layer F.Cu) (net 7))
 (segment (start 128.141999 56.291999) (end 129.69 57.84) (width 0.5) (layer B.Cu) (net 10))
 (segment (start 123.323788 56.291999) (end 128.141999 56.291999) (width 0.5) (layer B.Cu) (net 10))
 (segment (start 123.19 56.425787) (end 123.323788 56.291999) (width 0.5) (layer B.Cu) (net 10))
 (segment (start 123.19 57.84) (end 123.19 56.425787) (width 0.5) (layer B.Cu) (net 10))
 (segment (start 130.9136 57.84) (end 132.3848 56.3688) (width 0.5) (layer F.Cu) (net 10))
 (segment (start 129.69 57.84) (end 130.9136 57.84) (width 0.5) (layer F.Cu) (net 10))
 (segment (start 122.991 57.84) (end 123.19 57.84) (width 0.5) (layer B.Cu) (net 10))
 (segment (start 119.0625 53.9115) (end 122.991 57.84) (width 0.5) (layer B.Cu) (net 10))
 (segment (start 132.939998 93.66) (end 133.32 93.66) (width 0.5) (layer F.Cu) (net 10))
 (segment (start 131.719999 92.440001) (end 132.939998 93.66) (width 0.5) (layer F.Cu) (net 10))
 (segment (start 131.719999 75.905801) (end 131.719999 92.440001) (width 0.5) (layer F.Cu) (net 10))
 (segment (start 132.2578 75.368) (end 132.2578 75.368) (width 0.5) (layer F.Cu) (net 10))
 (segment (start 132.2578 75.368) (end 131.719999 75.905801) (width 0.5) (layer F.Cu) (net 10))
 (via (at 132.2578 75.368) (size 0.8) (drill 0.4) (layers F.Cu B.Cu) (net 10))
 (segment (start 131.346508 73.04183) (end 125.233678 66.929) (width 0.5) (layer B.Cu) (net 10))
 (segment (start 131.346508 73.206708) (end 131.346508 73.04183) (width 0.5) (layer B.Cu) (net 10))
 (segment (start 132.2578 74.118) (end 131.346508 73.206708) (width 0.5) (layer B.Cu) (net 10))
 (segment (start 132.2578 75.368) (end 132.2578 74.118) (width 0.5) (layer B.Cu) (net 10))
 (segment (start 125.233678 66.929) (end 119.126 66.929) (width 0.5) (layer B.Cu) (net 10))
 (segment (start 117.862499 65.665499) (end 117.862499 55.111501) (width 0.5) (layer B.Cu) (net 10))
 (segment (start 117.862499 55.111501) (end 119.0625 53.9115) (width 0.5) (layer B.Cu) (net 10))
 (segment (start 119.126 66.929) (end 117.862499 65.665499) (width 0.5) (layer B.Cu) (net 10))
 (segment (start 117.446491 77.986491) (end 118.12 78.66) (width 0.5) (layer F.Cu) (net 2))
 (segment (start 119.0625 58.9915) (end 117.262488 60.791512) (width 0.5) (layer F.Cu) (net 2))
 (segment (start 117.262488 60.791512) (end 117.262488 65.779431) (width 0.5) (layer F.Cu) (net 2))
 (segment (start 117.262488 65.779431) (end 117.446491 65.963434) (width 0.5) (layer F.Cu) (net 2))
 (segment (start 117.446491 65.963434) (end 117.446491 77.986491) (width 0.5) (layer F.Cu) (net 2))
 (segment (start 118.12 78.66) (end 118.12 79.66) (width 0.5) (layer F.Cu) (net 2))
 (segment (start 119.0625 56.4515) (end 116.332 59.182) (width 0.5) (layer F.Cu) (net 1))
 (segment (start 116.332 59.182) (end 116.332 80.9625) (width 0.5) (layer F.Cu) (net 1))
 (segment (start 117.0295 81.66) (end 118.12 81.66) (width 0.5) (layer F.Cu) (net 1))
 (segment (start 116.332 80.9625) (end 117.0295 81.66) (width 0.5) (layer F.Cu) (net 1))
 (segment (start 134.920001 75.922001) (end 134.920001 88.599999) (width 0.5) (layer F.Cu) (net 9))
 (segment (start 134.4168 75.4188) (end 134.920001 75.922001) (width 0.5) (layer F.Cu) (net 9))
 (segment (start 133.86 89.66) (end 133.32 89.66) (width 0.5) (layer F.Cu) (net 9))
 (segment (start 134.920001 88.599999) (end 133.86 89.66) (width 0.5) (layer F.Cu) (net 9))
 (segment (start 127.7874 77.0926) (end 126.72 78.16) (width 0.5) (layer F.Cu) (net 5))
 (segment (start 127.7874 75.3488) (end 127.7874 77.0926) (width 0.5) (layer F.Cu) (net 5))
 (segment (start 125.5268 77.3532) (end 124.72 78.16) (width 0.5) (layer F.Cu) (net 4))
 (segment (start 125.5268 75.368) (end 125.5268 77.3532) (width 0.5) (layer F.Cu) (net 4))
 (segment (start 124.426799 74.267999) (end 125.5268 75.368) (width 0.5) (layer F.Cu) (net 4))
 (segment (start 124.426799 72.277997) (end 124.426799 74.267999) (width 0.5) (layer F.Cu) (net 4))
 (segment (start 124.067601 71.918799) (end 124.426799 72.277997) (width 0.5) (layer F.Cu) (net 4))
 (segment (start 120.163601 71.918799) (end 124.067601 71.918799) (width 0.5) (layer F.Cu) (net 4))
 (segment (start 119.507 72.5754) (end 120.163601 71.918799) (width 0.5) (layer F.Cu) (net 4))
 (via (at 125.7935 63.3095) (size 0.8) (drill 0.4) (layers F.Cu B.Cu) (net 11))
 (via (at 124.714 64.7065) (size 0.8) (drill 0.4) (layers F.Cu B.Cu) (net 11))
 (via (at 125.7935 64.77) (size 0.8) (drill 0.4) (layers F.Cu B.Cu) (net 11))
 (via (at 126.9365 64.643) (size 0.8) (drill 0.4) (layers F.Cu B.Cu) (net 11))
 (via (at 126.9365 63.373) (size 0.8) (drill 0.4) (layers F.Cu B.Cu) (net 11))
 (via (at 124.6505 63.3095) (size 0.8) (drill 0.4) (layers F.Cu B.Cu) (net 11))
 (segment (start 134.62 57.38) (end 132.75 59.25) (width 0.5) (layer B.Cu) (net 11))
 (segment (start 134.62 55.88) (end 134.62 57.38) (width 0.5) (layer B.Cu) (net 11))
 (segment (start 132.75 61.284) (end 132.9334 61.4674) (width 0.5) (layer B.Cu) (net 11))
 (segment (start 132.75 59.25) (end 132.75 61.284) (width 0.5) (layer B.Cu) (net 11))
 (segment (start 134.62 56.263602) (end 134.62 55.88) (width 0.5) (layer F.Cu) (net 11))
 (segment (start 126.9365 63.373) (end 127.510602 63.373) (width 0.5) (layer F.Cu) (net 11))
 (segment (start 130.208051 60.675551) (end 134.62 56.263602) (width 0.5) (layer F.Cu) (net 11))
 (segment (start 127.510602 63.373) (end 130.208051 60.675551) (width 0.5) (layer F.Cu) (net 11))
 (segment (start 131.38408 63.01672) (end 131.38408 63.82064) (width 0.5) (layer B.Cu) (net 11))
 (segment (start 132.9334 61.4674) (end 131.38408 63.01672) (width 0.5) (layer B.Cu) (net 11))
 (segment (start 135.3185 64.192) (end 131.6925 64.192) (width 0.5) (layer F.Cu) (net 11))
 (segment (start 131.6925 64.192) (end 131.445 63.9445) (width 0.5) (layer F.Cu) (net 11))
 (segment (start 131.38408 63.82064) (end 131.38408 63.82064) (width 0.5) (layer B.Cu) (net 11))
 (via (at 131.38408 63.82064) (size 0.8) (drill 0.4) (layers F.Cu B.Cu) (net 11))
 (segment (start 126.238 53.975) (end 128.135 53.975) (width 0.5) (layer B.Cu) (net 11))
 (segment (start 128.135 53.975) (end 132.75 58.59) (width 0.5) (layer B.Cu) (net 11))
 (segment (start 132.75 58.59) (end 132.75 59.25) (width 0.5) (layer B.Cu) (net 11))
 (segment (start 128.127639 59.420639) (end 126.238 57.531) (width 0.5) (layer B.Cu) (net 12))
 (segment (start 130.034079 59.420639) (end 128.127639 59.420639) (width 0.5) (layer B.Cu) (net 12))
 (segment (start 131.38408 60.77064) (end 130.034079 59.420639) (width 0.5) (layer B.Cu) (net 12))
 (segment (start 130.048 76.832) (end 128.72 78.16) (width 0.5) (layer F.Cu) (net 6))
 (segment (start 130.048 75.3488) (end 130.048 76.832) (width 0.5) (layer F.Cu) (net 6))
 (segment (start 132.328399 63.167399) (end 132.1435 63.352298) (width 0.5) (layer B.Cu) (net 13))
 (segment (start 134.003393 63.167399) (end 132.328399 63.167399) (width 0.5) (layer B.Cu) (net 13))
 (segment (start 135.001 62.169792) (end 134.003393 63.167399) (width 0.5) (layer B.Cu) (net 13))
 (segment (start 135.001 61.468) (end 135.001 62.169792) (width 0.5) (layer B.Cu) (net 13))
 (segment (start 129.48408 64.690632) (end 129.48408 63.82064) (width 0.5) (layer B.Cu) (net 13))
 (segment (start 129.964098 65.17065) (end 129.48408 64.690632) (width 0.5) (layer B.Cu) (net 13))
 (segment (start 131.989072 65.17065) (end 129.964098 65.17065) (width 0.5) (layer B.Cu) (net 13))
 (segment (start 132.1435 65.016222) (end 131.989072 65.17065) (width 0.5) (layer B.Cu) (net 13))
 (segment (start 132.1435 63.352298) (end 132.1435 65.016222) (width 0.5) (layer B.Cu) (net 13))
 (segment (start 120.8216 75.2348) (end 123.0376 73.0188) (width 0.5) (layer F.Cu) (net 14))
 (segment (start 120.4187 75.2348) (end 120.8216 75.2348) (width 0.5) (layer F.Cu) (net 14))
 (segment (start 123.0376 75.8424) (end 120.72 78.16) (width 0.5) (layer F.Cu) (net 3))
 (segment (start 123.0376 75.4188) (end 123.0376 75.8424) (width 0.5) (layer F.Cu) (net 3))
 (segment (start 134.6074 51.8922) (end 135.4074 51.8922) (width 0.5) (layer F.Cu) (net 15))
 (segment (start 132.5308 53.9688) (end 134.6074 51.8922) (width 0.5) (layer F.Cu) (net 15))
 (segment (start 132.3848 53.9688) (end 132.5308 53.9688) (width 0.5) (layer F.Cu) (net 15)))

